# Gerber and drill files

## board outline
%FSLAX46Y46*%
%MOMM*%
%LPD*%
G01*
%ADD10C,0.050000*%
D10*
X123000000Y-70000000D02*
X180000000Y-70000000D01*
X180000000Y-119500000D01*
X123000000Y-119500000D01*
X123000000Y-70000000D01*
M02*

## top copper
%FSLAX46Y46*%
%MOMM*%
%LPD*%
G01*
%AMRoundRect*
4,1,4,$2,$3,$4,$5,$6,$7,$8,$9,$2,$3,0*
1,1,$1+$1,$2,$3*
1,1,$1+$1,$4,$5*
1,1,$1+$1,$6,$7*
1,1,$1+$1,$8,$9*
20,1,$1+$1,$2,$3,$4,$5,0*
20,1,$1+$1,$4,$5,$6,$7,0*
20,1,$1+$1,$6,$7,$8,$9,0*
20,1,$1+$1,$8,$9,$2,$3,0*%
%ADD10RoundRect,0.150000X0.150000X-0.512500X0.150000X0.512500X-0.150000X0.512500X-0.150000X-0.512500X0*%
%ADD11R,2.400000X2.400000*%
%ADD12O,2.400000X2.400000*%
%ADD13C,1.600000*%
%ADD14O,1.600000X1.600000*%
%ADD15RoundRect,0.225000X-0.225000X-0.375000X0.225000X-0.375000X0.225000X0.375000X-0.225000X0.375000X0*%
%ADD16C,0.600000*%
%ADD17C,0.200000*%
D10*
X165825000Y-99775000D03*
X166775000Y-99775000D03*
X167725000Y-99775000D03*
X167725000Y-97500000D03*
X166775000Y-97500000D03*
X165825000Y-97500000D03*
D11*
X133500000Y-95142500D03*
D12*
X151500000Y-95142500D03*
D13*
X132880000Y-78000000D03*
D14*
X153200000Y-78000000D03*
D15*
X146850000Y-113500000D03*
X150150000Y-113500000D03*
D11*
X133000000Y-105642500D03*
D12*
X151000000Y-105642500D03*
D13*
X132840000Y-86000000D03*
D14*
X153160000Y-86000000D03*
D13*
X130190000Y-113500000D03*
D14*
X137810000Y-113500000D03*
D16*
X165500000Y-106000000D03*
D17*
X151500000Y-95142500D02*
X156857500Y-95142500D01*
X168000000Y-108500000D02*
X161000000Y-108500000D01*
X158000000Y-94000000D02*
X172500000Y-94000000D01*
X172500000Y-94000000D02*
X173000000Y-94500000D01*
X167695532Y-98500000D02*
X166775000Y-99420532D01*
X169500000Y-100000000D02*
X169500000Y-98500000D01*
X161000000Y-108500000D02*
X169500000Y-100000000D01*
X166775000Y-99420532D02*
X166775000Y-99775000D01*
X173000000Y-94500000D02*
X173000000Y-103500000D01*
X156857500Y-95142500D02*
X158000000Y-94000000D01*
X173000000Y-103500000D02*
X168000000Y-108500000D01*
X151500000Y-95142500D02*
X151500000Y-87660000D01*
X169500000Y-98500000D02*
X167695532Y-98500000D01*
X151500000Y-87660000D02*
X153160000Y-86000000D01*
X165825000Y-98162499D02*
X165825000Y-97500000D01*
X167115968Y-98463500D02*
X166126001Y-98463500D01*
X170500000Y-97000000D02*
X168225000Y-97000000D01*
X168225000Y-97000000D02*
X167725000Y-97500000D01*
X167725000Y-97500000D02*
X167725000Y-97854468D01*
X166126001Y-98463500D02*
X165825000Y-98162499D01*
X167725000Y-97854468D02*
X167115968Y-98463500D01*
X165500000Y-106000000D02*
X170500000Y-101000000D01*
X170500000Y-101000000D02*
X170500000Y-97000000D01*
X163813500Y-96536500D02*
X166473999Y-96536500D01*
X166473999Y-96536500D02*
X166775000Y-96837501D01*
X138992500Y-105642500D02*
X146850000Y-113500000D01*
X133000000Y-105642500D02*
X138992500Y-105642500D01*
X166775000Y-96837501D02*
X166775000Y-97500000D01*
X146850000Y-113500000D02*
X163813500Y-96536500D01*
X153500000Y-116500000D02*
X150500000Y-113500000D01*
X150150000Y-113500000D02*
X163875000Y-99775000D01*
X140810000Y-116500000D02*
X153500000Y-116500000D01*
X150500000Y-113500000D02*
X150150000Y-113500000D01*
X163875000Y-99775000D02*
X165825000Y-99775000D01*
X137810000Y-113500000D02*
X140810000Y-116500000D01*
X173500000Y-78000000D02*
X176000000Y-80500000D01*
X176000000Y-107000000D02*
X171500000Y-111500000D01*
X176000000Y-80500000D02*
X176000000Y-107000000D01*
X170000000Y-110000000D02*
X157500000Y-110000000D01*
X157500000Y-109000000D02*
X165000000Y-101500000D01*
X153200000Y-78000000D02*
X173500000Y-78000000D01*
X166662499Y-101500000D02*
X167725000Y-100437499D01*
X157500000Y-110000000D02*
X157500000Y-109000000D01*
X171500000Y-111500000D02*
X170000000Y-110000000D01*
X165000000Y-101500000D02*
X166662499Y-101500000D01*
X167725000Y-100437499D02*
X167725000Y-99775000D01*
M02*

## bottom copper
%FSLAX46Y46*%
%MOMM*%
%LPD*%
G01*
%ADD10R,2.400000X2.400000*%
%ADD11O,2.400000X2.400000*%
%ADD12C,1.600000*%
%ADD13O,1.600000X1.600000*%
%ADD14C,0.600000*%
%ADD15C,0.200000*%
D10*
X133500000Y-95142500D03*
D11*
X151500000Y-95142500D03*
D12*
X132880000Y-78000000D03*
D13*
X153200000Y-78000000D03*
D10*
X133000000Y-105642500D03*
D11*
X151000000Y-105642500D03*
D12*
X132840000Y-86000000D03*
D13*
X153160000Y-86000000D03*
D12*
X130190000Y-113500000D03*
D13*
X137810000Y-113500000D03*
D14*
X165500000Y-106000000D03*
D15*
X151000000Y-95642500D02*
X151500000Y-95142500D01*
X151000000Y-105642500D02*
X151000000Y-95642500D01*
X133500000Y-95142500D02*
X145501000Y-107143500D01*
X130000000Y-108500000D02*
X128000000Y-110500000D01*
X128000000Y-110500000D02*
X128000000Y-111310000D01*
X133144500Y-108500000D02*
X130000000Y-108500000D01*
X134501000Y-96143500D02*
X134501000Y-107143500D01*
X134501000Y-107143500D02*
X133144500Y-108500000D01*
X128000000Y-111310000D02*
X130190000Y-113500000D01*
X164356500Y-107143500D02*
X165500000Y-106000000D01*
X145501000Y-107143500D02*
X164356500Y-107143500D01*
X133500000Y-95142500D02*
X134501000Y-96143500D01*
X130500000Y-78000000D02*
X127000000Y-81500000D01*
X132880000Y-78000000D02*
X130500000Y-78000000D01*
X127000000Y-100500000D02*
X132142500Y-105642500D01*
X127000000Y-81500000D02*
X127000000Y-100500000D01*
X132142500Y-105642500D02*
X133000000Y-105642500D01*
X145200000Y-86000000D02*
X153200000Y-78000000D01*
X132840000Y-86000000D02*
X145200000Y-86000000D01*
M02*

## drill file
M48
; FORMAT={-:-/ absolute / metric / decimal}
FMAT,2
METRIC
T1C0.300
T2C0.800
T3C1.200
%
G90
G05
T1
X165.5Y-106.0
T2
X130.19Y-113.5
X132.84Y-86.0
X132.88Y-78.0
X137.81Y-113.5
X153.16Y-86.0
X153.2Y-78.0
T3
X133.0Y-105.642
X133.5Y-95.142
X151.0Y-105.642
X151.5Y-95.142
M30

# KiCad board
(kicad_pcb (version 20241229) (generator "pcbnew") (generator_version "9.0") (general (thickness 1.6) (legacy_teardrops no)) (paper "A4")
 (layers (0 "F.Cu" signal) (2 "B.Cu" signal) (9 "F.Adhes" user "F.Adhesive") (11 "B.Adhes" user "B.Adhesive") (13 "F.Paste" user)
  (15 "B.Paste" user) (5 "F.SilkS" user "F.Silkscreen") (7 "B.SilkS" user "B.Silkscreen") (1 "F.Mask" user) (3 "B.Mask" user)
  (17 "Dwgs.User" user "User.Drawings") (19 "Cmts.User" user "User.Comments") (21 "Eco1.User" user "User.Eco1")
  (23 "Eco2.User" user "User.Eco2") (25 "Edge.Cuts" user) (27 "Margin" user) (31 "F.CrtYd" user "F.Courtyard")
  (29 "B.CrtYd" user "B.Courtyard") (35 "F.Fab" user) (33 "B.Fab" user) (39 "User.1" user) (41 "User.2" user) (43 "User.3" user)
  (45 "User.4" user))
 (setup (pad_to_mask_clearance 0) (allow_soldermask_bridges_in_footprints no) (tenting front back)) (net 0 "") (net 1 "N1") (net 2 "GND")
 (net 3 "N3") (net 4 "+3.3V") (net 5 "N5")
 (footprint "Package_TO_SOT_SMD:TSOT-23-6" (layer "F.Cu") (at 166.775 98.6375 90)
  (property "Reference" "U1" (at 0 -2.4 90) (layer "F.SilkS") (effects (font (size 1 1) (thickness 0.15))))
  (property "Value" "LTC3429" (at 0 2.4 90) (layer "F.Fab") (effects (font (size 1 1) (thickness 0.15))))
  (pad "1" smd roundrect (at -1.1375 -0.95 90) (size 1.325 0.6) (layers "F.Cu" "F.Mask" "F.Paste") (roundrect_rratio 0.25) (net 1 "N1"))
  (pad "2" smd roundrect (at -1.1375 0 90) (size 1.325 0.6) (layers "F.Cu" "F.Mask" "F.Paste") (roundrect_rratio 0.25) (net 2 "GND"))
  (pad "3" smd roundrect (at -1.1375 0.95 90) (size 1.325 0.6) (layers "F.Cu" "F.Mask" "F.Paste") (roundrect_rratio 0.25) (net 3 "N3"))
  (pad "4" smd roundrect (at 1.1375 0.95 90) (size 1.325 0.6) (layers "F.Cu" "F.Mask" "F.Paste") (roundrect_rratio 0.25) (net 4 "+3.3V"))
  (pad "5" smd roundrect (at 1.1375 0 90) (size 1.325 0.6) (layers "F.Cu" "F.Mask" "F.Paste") (roundrect_rratio 0.25) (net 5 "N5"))
  (pad "6" smd roundrect (at 1.1375 -0.95 90) (size 1.325 0.6) (layers "F.Cu" "F.Mask" "F.Paste") (roundrect_rratio 0.25) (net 4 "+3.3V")))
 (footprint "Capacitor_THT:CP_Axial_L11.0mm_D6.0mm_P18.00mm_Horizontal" (layer "F.Cu") (at 133.5 95.1425)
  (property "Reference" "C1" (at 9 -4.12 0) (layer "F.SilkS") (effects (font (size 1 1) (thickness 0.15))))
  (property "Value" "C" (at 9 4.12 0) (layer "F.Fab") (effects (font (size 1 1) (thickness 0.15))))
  (pad "1" thru_hole rect (at 0 0) (size 2.4 2.4) (drill 1.2) (layers "*.Cu" "*.Mask") (remove_unused_layers no) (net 4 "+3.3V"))
  (pad "2" thru_hole oval (at 18 0) (size 2.4 2.4) (drill 1.2) (layers "*.Cu" "*.Mask") (remove_unused_layers no) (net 2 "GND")))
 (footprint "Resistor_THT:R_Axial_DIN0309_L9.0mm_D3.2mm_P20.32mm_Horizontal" (layer "F.Cu") (at 132.88 78)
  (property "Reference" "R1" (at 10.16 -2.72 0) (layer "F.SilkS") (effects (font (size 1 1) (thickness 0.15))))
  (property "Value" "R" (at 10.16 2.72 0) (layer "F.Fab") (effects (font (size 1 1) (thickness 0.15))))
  (pad "1" thru_hole circle (at 0 0) (size 1.6 1.6) (drill 0.8) (layers "*.Cu" "*.Mask") (remove_unused_layers no) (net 5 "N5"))
  (pad "2" thru_hole oval (at 20.32 0) (size 1.6 1.6) (drill 0.8) (layers "*.Cu" "*.Mask") (remove_unused_layers no) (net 3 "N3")))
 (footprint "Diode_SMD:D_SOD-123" (layer "F.Cu") (at 148.5 113.5)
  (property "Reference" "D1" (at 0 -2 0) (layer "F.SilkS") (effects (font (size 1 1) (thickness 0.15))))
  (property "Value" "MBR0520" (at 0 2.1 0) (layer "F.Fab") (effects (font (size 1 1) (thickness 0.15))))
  (pad "1" smd roundrect (at -1.65 0) (size 0.9 1.2) (layers "F.Cu" "F.Mask" "F.Paste") (roundrect_rratio 0.25) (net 5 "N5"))
  (pad "2" smd roundrect (at 1.65 0) (size 0.9 1.2) (layers "F.Cu" "F.Mask" "F.Paste") (roundrect_rratio 0.25) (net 1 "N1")))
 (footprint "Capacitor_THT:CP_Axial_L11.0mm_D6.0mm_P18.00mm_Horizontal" (layer "F.Cu") (at 133 105.6425)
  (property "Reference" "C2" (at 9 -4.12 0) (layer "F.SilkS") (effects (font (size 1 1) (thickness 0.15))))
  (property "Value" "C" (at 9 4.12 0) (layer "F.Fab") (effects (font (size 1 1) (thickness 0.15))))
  (pad "1" thru_hole rect (at 0 0) (size 2.4 2.4) (drill 1.2) (layers "*.Cu" "*.Mask") (remove_unused_layers no) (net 5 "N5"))
  (pad "2" thru_hole oval (at 18 0) (size 2.4 2.4) (drill 1.2) (layers "*.Cu" "*.Mask") (remove_unused_layers no) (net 2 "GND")))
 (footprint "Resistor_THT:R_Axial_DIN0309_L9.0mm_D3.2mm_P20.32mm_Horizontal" (layer "F.Cu") (at 132.84 86)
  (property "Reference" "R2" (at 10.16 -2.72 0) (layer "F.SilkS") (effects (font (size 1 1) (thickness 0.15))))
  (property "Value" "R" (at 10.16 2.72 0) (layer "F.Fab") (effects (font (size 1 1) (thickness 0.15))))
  (pad "1" thru_hole circle (at 0 0) (size 1.6 1.6) (drill 0.8) (layers "*.Cu" "*.Mask") (remove_unused_layers no) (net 3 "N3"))
  (pad "2" thru_hole oval (at 20.32 0) (size 1.6 1.6) (drill 0.8) (layers "*.Cu" "*.Mask") (remove_unused_layers no) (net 2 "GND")))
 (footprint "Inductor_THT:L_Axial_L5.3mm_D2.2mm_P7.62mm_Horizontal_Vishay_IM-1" (layer "F.Cu") (at 130.19 113.5)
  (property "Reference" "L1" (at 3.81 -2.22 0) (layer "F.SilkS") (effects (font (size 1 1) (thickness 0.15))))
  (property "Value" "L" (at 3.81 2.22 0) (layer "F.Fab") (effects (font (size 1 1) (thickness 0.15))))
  (pad "1" thru_hole circle (at 0 0) (size 1.6 1.6) (drill 0.8) (layers "*.Cu" "*.Mask") (remove_unused_layers no) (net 4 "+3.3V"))
  (pad "2" thru_hole oval (at 7.62 0) (size 1.6 1.6) (drill 0.8) (layers "*.Cu" "*.Mask") (remove_unused_layers no) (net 1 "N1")))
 (gr_rect (start 123 70) (end 180 119.5) (stroke (width 0.05) (type default)) (fill no) (layer "Edge.Cuts"))
 (segment (start 151.5 95.1425) (end 156.8575 95.1425) (width 0.2) (layer "F.Cu") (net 2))
 (segment (start 168 108.5) (end 161 108.5) (width 0.2) (layer "F.Cu") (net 2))
 (segment (start 158 94) (end 172.5 94) (width 0.2) (layer "F.Cu") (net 2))
 (segment (start 172.5 94) (end 173 94.5) (width 0.2) (layer "F.Cu") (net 2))
 (segment (start 167.695532 98.5) (end 166.775 99.420532) (width 0.2) (layer "F.Cu") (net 2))
 (segment (start 169.5 100) (end 169.5 98.5) (width 0.2) (layer "F.Cu") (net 2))
 (segment (start 161 108.5) (end 169.5 100) (width 0.2) (layer "F.Cu") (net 2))
 (segment (start 166.775 99.420532) (end 166.775 99.775) (width 0.2) (layer "F.Cu") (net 2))
 (segment (start 173 94.5) (end 173 103.5) (width 0.2) (layer "F.Cu") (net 2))
 (segment (start 156.8575 95.1425) (end 158 94) (width 0.2) (layer "F.Cu") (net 2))
 (segment (start 173 103.5) (end 168 108.5) (width 0.2) (layer "F.Cu") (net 2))
 (segment (start 151.5 95.1425) (end 151.5 87.66) (width 0.2) (layer "F.Cu") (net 2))
 (segment (start 169.5 98.5) (end 167.695532 98.5) (width 0.2) (layer "F.Cu") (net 2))
 (segment (start 151.5 87.66) (end 153.16 86) (width 0.2) (layer "F.Cu") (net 2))
 (segment (start 151 95.6425) (end 151.5 95.1425) (width 0.2) (layer "B.Cu") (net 2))
 (segment (start 151 105.6425) (end 151 95.6425) (width 0.2) (layer "B.Cu") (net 2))
 (segment (start 165.825 98.162499) (end 165.825 97.5) (width 0.2) (layer "F.Cu") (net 4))
 (segment (start 167.115968 98.4635) (end 166.126001 98.4635) (width 0.2) (layer "F.Cu") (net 4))
 (segment (start 170.5 97) (end 168.225 97) (width 0.2) (layer "F.Cu") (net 4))
 (segment (start 168.225 97) (end 167.725 97.5) (width 0.2) (layer "F.Cu") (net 4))
 (segment (start 167.725 97.5) (end 167.725 97.854468) (width 0.2) (layer "F.Cu") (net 4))
 (segment (start 166.126001 98.4635) (end 165.825 98.162499) (width 0.2) (layer "F.Cu") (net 4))
 (segment (start 167.725 97.854468) (end 167.115968 98.4635) (width 0.2) (layer "F.Cu") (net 4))
 (segment (start 165.5 106) (end 170.5 101) (width 0.2) (layer "F.Cu") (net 4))
 (segment (start 170.5 101) (end 170.5 97) (width 0.2) (layer "F.Cu") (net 4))
 (via (at 165.5 106) (size 0.6) (drill 0.3) (layers "F.Cu" "B.Cu") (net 4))
 (segment (start 133.5 95.1425) (end 145.501 107.1435) (width 0.2) (layer "B.Cu") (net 4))
 (segment (start 130 108.5) (end 128 110.5) (width 0.2) (layer "B.Cu") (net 4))
 (segment (start 128 110.5) (end 128 111.31) (width 0.2) (layer "B.Cu") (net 4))
 (segment (start 133.1445 108.5) (end 130 108.5) (width 0.2) (layer "B.Cu") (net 4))
 (segment (start 134.501 96.1435) (end 134.501 107.1435) (width 0.2) (layer "B.Cu") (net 4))
 (segment (start 134.501 107.1435) (end 133.1445 108.5) (width 0.2) (layer "B.Cu") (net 4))
 (segment (start 128 111.31) (end 130.19 113.5) (width 0.2) (layer "B.Cu") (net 4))
 (segment (start 164.3565 107.1435) (end 165.5 106) (width 0.2) (layer "B.Cu") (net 4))
 (segment (start 145.501 107.1435) (end 164.3565 107.1435) (width 0.2) (layer "B.Cu") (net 4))
 (segment (start 133.5 95.1425) (end 134.501 96.1435) (width 0.2) (layer "B.Cu") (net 4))
 (segment (start 163.8135 96.5365) (end 166.473999 96.5365) (width 0.2) (layer "F.Cu") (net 5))
 (segment (start 166.473999 96.5365) (end 166.775 96.837501) (width 0.2) (layer "F.Cu") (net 5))
 (segment (start 138.9925 105.6425) (end 146.85 113.5) (width 0.2) (layer "F.Cu") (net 5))
 (segment (start 133 105.6425) (end 138.9925 105.6425) (width 0.2) (layer "F.Cu") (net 5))
 (segment (start 166.775 96.837501) (end 166.775 97.5) (width 0.2) (layer "F.Cu") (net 5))
 (segment (start 146.85 113.5) (end 163.8135 96.5365) (width 0.2) (layer "F.Cu") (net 5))
 (segment (start 130.5 78) (end 127 81.5) (width 0.2) (layer "B.Cu") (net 5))
 (segment (start 132.88 78) (end 130.5 78) (width 0.2) (layer "B.Cu") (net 5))
 (segment (start 127 100.5) (end 132.1425 105.6425) (width 0.2) (layer "B.Cu") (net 5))
 (segment (start 127 81.5) (end 127 100.5) (width 0.2) (layer "B.Cu") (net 5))
 (segment (start 132.1425 105.6425) (end 133 105.6425) (width 0.2) (layer "B.Cu") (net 5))
 (segment (start 153.5 116.5) (end 150.5 113.5) (width 0.2) (layer "F.Cu") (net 1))
 (segment (start 150.15 113.5) (end 163.875 99.775) (width 0.2) (layer "F.Cu") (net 1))
 (segment (start 140.81 116.5) (end 153.5 116.5) (width 0.2) (layer "F.Cu") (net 1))
 (segment (start 150.5 113.5) (end 150.15 113.5) (width 0.2) (layer "F.Cu") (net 1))
 (segment (start 163.875 99.775) (end 165.825 99.775) (width 0.2) (layer "F.Cu") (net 1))
 (segment (start 137.81 113.5) (end 140.81 116.5) (width 0.2) (layer "F.Cu") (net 1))
 (segment (start 173.5 78) (end 176 80.5) (width 0.2) (layer "F.Cu") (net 3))
 (segment (start 176 107) (end 171.5 111.5) (width 0.2) (layer "F.Cu") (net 3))
 (segment (start 176 80.5) (end 176 107) (width 0.2) (layer "F.Cu") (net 3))
 (segment (start 170 110) (end 157.5 110) (width 0.2) (layer "F.Cu") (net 3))
 (segment (start 157.5 109) (end 165 101.5) (width 0.2) (layer "F.Cu") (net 3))
 (segment (start 153.2 78) (end 173.5 78) (width 0.2) (layer "F.Cu") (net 3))
 (segment (start 166.662499 101.5) (end 167.725 100.437499) (width 0.2) (layer "F.Cu") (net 3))
 (segment (start 157.5 110) (end 157.5 109) (width 0.2) (layer "F.Cu") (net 3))
 (segment (start 171.5 111.5) (end 170 110) (width 0.2) (layer "F.Cu") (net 3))
 (segment (start 165 101.5) (end 166.662499 101.5) (width 0.2) (layer "F.Cu") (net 3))
 (segment (start 167.725 100.437499) (end 167.725 99.775) (width 0.2) (layer "F.Cu") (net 3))
 (segment (start 145.2 86) (end 153.2 78) (width 0.2) (layer "B.Cu") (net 3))
 (segment (start 132.84 86) (end 145.2 86) (width 0.2) (layer "B.Cu") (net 3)))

